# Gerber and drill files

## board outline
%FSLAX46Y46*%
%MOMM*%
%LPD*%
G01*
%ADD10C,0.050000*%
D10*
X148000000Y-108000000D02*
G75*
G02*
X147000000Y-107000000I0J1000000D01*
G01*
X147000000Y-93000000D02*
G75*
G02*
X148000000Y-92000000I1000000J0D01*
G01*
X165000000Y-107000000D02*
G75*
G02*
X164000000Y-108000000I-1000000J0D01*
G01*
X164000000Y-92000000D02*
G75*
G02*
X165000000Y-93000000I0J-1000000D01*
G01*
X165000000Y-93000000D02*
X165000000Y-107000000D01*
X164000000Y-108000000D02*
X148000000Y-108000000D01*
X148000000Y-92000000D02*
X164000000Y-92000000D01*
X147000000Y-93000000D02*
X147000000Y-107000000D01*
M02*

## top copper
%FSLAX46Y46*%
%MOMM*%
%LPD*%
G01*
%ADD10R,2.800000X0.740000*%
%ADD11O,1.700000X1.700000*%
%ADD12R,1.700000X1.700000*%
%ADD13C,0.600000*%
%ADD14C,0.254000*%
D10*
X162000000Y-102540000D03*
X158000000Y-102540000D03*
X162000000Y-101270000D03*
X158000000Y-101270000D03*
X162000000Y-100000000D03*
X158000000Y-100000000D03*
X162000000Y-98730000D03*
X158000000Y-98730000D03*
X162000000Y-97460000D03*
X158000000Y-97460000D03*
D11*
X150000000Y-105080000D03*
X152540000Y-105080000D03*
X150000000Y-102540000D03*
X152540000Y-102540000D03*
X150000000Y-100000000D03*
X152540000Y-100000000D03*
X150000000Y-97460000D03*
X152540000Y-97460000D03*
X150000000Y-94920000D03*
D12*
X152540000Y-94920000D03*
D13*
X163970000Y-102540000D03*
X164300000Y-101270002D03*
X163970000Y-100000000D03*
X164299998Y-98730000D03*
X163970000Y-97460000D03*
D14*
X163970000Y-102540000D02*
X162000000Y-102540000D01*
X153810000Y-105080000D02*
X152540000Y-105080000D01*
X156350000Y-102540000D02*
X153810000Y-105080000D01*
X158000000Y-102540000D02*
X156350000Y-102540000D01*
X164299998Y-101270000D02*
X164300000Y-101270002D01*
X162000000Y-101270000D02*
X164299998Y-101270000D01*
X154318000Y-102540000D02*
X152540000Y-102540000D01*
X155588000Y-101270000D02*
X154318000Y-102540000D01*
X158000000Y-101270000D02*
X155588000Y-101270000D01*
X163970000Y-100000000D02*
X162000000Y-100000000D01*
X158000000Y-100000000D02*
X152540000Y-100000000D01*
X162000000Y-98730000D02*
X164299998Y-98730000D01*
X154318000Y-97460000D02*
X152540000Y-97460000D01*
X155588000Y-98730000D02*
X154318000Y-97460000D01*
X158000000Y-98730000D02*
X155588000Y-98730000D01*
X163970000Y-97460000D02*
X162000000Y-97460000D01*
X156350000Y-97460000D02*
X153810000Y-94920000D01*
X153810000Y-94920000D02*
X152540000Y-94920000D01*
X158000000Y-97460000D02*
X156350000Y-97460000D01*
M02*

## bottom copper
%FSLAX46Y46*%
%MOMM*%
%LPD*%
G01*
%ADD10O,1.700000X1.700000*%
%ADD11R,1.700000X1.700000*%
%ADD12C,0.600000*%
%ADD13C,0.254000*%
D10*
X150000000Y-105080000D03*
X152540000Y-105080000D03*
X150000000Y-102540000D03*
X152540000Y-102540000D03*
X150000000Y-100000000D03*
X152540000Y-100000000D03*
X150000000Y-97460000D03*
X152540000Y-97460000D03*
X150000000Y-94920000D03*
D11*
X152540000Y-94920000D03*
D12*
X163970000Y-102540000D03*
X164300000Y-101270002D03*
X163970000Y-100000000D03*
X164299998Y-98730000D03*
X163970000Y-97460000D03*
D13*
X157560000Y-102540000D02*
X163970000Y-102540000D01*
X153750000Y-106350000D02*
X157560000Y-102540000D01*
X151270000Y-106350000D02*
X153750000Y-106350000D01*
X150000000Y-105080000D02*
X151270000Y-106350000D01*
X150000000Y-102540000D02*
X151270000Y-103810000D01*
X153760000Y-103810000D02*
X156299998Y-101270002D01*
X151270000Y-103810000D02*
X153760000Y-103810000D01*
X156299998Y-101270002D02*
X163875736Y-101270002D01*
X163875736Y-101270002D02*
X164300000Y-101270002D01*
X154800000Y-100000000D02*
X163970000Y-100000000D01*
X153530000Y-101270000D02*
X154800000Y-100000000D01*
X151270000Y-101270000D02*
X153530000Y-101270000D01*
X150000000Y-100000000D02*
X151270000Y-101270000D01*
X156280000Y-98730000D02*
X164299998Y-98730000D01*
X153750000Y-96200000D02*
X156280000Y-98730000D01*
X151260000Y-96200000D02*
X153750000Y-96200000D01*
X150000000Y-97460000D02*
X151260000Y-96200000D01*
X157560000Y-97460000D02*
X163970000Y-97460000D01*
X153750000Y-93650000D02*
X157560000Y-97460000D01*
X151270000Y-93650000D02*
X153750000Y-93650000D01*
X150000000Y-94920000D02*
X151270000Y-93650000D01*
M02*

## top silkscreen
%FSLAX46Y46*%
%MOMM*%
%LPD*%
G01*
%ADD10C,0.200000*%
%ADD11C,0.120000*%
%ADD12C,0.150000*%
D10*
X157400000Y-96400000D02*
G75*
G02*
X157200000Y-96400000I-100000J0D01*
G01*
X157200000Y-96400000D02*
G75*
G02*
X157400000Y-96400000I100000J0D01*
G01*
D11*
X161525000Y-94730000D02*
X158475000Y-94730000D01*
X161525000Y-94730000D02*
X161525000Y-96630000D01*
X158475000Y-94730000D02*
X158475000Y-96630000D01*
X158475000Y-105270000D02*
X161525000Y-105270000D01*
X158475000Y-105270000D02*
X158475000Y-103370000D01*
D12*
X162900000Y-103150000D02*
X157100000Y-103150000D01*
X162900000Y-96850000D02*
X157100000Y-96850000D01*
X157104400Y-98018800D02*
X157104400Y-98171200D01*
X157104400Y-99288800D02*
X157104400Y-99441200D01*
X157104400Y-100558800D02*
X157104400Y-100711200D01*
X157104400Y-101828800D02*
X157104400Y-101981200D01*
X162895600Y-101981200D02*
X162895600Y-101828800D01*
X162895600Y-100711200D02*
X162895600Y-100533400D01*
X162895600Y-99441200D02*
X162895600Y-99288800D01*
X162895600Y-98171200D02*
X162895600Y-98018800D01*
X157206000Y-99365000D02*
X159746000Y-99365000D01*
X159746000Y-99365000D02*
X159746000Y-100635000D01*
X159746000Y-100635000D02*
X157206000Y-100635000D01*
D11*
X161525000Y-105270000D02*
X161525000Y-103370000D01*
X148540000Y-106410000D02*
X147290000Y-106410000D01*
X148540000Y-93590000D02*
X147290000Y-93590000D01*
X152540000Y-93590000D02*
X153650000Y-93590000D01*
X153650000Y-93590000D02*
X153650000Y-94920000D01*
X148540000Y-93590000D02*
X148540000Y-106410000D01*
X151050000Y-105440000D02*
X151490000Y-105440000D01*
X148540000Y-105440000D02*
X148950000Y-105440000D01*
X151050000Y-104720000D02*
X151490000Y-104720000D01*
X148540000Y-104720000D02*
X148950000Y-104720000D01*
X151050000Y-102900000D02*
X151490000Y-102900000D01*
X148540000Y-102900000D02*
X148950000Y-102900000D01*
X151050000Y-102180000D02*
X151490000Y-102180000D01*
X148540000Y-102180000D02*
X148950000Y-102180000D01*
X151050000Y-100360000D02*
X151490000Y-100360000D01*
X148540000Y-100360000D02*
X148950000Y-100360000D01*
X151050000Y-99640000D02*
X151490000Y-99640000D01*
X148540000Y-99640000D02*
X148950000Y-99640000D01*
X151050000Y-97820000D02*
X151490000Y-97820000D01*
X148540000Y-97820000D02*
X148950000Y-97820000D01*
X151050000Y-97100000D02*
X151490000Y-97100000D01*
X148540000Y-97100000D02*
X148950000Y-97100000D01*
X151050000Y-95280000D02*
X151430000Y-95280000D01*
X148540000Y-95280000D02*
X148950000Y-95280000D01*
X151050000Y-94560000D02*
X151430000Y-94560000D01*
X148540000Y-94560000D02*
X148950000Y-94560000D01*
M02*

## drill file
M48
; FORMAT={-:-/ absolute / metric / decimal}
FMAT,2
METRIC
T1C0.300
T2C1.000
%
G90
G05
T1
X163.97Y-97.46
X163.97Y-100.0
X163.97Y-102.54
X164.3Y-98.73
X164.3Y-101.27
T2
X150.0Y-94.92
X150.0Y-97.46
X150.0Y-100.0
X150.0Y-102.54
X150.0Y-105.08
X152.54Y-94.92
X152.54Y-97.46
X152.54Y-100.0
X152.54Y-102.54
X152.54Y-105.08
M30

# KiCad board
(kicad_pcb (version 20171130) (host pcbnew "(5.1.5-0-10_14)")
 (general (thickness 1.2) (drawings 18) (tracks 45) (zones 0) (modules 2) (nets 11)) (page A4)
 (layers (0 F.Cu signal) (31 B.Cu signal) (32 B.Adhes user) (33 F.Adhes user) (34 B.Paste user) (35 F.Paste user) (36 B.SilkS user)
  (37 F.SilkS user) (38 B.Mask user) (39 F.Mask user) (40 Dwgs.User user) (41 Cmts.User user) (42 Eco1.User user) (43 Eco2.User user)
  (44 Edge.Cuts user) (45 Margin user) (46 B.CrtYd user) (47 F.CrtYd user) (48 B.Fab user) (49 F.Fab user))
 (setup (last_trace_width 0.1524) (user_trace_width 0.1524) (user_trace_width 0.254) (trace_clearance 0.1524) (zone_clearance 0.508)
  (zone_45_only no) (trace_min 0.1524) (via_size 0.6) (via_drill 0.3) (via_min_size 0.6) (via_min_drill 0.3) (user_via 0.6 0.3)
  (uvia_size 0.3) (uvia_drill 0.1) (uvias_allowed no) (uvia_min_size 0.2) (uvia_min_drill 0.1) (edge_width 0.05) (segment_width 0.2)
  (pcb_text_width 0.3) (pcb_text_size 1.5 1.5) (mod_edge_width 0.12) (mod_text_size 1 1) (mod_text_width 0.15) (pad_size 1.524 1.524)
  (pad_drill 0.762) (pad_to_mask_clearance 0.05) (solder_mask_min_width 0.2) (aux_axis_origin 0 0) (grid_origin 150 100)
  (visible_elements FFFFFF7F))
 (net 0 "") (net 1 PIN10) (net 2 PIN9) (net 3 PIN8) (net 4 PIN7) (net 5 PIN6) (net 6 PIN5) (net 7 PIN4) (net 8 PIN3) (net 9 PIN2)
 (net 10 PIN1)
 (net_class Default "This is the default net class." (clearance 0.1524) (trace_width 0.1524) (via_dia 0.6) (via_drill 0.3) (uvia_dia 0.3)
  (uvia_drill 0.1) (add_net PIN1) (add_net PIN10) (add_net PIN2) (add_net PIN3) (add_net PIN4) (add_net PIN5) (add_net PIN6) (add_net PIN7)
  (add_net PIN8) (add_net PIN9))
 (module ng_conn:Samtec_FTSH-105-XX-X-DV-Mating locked (layer F.Cu) (at 160 100 90)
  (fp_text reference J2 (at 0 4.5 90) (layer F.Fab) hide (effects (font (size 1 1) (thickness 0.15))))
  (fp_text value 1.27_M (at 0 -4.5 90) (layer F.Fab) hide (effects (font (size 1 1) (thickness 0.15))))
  (fp_circle (center 3.6 -2.7) (end 3.7 -2.7) (layer F.SilkS) (width 0.2))
  (fp_line (start 5.27 1.525) (end 5.27 -1.525) (layer F.SilkS) (width 0.12))
  (fp_line (start 5.27 1.525) (end 3.37 1.525) (layer F.SilkS) (width 0.12))
  (fp_line (start 5.27 -1.525) (end 3.37 -1.525) (layer F.SilkS) (width 0.12))
  (fp_line (start -5.27 -1.525) (end -5.27 1.525) (layer F.SilkS) (width 0.12))
  (fp_line (start -5.27 -1.525) (end -3.37 -1.525) (layer F.SilkS) (width 0.12))
  (fp_line (start -3.15 2.9) (end -3.15 -2.9) (layer F.SilkS) (width 0.15))
  (fp_line (start 3.15 2.9) (end 3.15 -2.9) (layer F.SilkS) (width 0.15))
  (fp_line (start 1.9812 -2.8956) (end 1.8288 -2.8956) (layer F.SilkS) (width 0.15))
  (fp_line (start 0.7112 -2.8956) (end 0.5588 -2.8956) (layer F.SilkS) (width 0.15))
  (fp_line (start -0.5588 -2.8956) (end -0.7112 -2.8956) (layer F.SilkS) (width 0.15))
  (fp_line (start -1.8288 -2.8956) (end -1.9812 -2.8956) (layer F.SilkS) (width 0.15))
  (fp_line (start -1.9812 2.8956) (end -1.8288 2.8956) (layer F.SilkS) (width 0.15))
  (fp_line (start -0.7112 2.8956) (end -0.5334 2.8956) (layer F.SilkS) (width 0.15))
  (fp_line (start 0.5588 2.8956) (end 0.7112 2.8956) (layer F.SilkS) (width 0.15))
  (fp_line (start 1.8288 2.8956) (end 1.9812 2.8956) (layer F.SilkS) (width 0.15))
  (fp_line (start 0.635 -2.794) (end 0.635 -0.254) (layer F.SilkS) (width 0.15))
  (fp_line (start 0.635 -0.254) (end -0.635 -0.254) (layer F.SilkS) (width 0.15))
  (fp_line (start -0.635 -0.254) (end -0.635 -2.794) (layer F.SilkS) (width 0.15))
  (fp_line (start -5.27 1.525) (end -3.37 1.525) (layer F.SilkS) (width 0.12))
  (pad 10 smd rect (at -2.54 2 270) (size 0.74 2.8) (layers F.Cu F.Paste F.Mask) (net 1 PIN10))
  (pad 9 smd rect (at -2.54 -2 270) (size 0.74 2.8) (layers F.Cu F.Paste F.Mask) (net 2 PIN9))
  (pad 8 smd rect (at -1.27 2 270) (size 0.74 2.8) (layers F.Cu F.Paste F.Mask) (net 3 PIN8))
  (pad 7 smd rect (at -1.27 -2 270) (size 0.74 2.8) (layers F.Cu F.Paste F.Mask) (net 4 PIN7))
  (pad 6 smd rect (at 0 2 270) (size 0.74 2.8) (layers F.Cu F.Paste F.Mask) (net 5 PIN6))
  (pad 5 smd rect (at 0 -2 270) (size 0.74 2.8) (layers F.Cu F.Paste F.Mask) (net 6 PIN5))
  (pad 4 smd rect (at 1.27 2 270) (size 0.74 2.8) (layers F.Cu F.Paste F.Mask) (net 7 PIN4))
  (pad 3 smd rect (at 1.27 -2 270) (size 0.74 2.8) (layers F.Cu F.Paste F.Mask) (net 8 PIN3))
  (pad 2 smd rect (at 2.54 2 270) (size 0.74 2.8) (layers F.Cu F.Paste F.Mask) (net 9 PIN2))
  (pad 1 smd rect (at 2.54 -2 270) (size 0.74 2.8) (layers F.Cu F.Paste F.Mask) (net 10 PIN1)))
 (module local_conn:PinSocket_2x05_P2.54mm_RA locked (layer F.Cu) (at 152.54 94.92)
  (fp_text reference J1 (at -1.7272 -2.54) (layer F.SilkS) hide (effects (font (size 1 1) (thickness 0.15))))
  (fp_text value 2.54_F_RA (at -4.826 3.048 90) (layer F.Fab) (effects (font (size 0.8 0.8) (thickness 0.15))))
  (fp_line (start -4 11.49) (end -5.25 11.49) (layer F.SilkS) (width 0.12))
  (fp_line (start -4 -1.33) (end -5.25 -1.33) (layer F.SilkS) (width 0.12))
  (fp_line (start 0 -1.33) (end 1.11 -1.33) (layer F.SilkS) (width 0.12))
  (fp_line (start 1.11 -1.33) (end 1.11 0) (layer F.SilkS) (width 0.12))
  (fp_line (start -4 -1.33) (end -4 11.49) (layer F.SilkS) (width 0.12))
  (fp_line (start -1.49 10.52) (end -1.05 10.52) (layer F.SilkS) (width 0.12))
  (fp_line (start -4 10.52) (end -3.59 10.52) (layer F.SilkS) (width 0.12))
  (fp_line (start -1.49 9.8) (end -1.05 9.8) (layer F.SilkS) (width 0.12))
  (fp_line (start -4 9.8) (end -3.59 9.8) (layer F.SilkS) (width 0.12))
  (fp_line (start -1.49 7.98) (end -1.05 7.98) (layer F.SilkS) (width 0.12))
  (fp_line (start -4 7.98) (end -3.59 7.98) (layer F.SilkS) (width 0.12))
  (fp_line (start -1.49 7.26) (end -1.05 7.26) (layer F.SilkS) (width 0.12))
  (fp_line (start -4 7.26) (end -3.59 7.26) (layer F.SilkS) (width 0.12))
  (fp_line (start -1.49 5.44) (end -1.05 5.44) (layer F.SilkS) (width 0.12))
  (fp_line (start -4 5.44) (end -3.59 5.44) (layer F.SilkS) (width 0.12))
  (fp_line (start -1.49 4.72) (end -1.05 4.72) (layer F.SilkS) (width 0.12))
  (fp_line (start -4 4.72) (end -3.59 4.72) (layer F.SilkS) (width 0.12))
  (fp_line (start -1.49 2.9) (end -1.05 2.9) (layer F.SilkS) (width 0.12))
  (fp_line (start -4 2.9) (end -3.59 2.9) (layer F.SilkS) (width 0.12))
  (fp_line (start -1.49 2.18) (end -1.05 2.18) (layer F.SilkS) (width 0.12))
  (fp_line (start -4 2.18) (end -3.59 2.18) (layer F.SilkS) (width 0.12))
  (fp_line (start -1.49 0.36) (end -1.11 0.36) (layer F.SilkS) (width 0.12))
  (fp_line (start -4 0.36) (end -3.59 0.36) (layer F.SilkS) (width 0.12))
  (fp_line (start -1.49 -0.36) (end -1.11 -0.36) (layer F.SilkS) (width 0.12))
  (fp_line (start -4 -0.36) (end -3.59 -0.36) (layer F.SilkS) (width 0.12))
  (pad 10 thru_hole oval (at -2.54 10.16) (size 1.7 1.7) (drill 1) (layers *.Cu *.Mask) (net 1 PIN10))
  (pad 9 thru_hole oval (at 0 10.16) (size 1.7 1.7) (drill 1) (layers *.Cu *.Mask) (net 2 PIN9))
  (pad 8 thru_hole oval (at -2.54 7.62) (size 1.7 1.7) (drill 1) (layers *.Cu *.Mask) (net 3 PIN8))
  (pad 7 thru_hole oval (at 0 7.62) (size 1.7 1.7) (drill 1) (layers *.Cu *.Mask) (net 4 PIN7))
  (pad 6 thru_hole oval (at -2.54 5.08) (size 1.7 1.7) (drill 1) (layers *.Cu *.Mask) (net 5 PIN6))
  (pad 5 thru_hole oval (at 0 5.08) (size 1.7 1.7) (drill 1) (layers *.Cu *.Mask) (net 6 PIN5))
  (pad 4 thru_hole oval (at -2.54 2.54) (size 1.7 1.7) (drill 1) (layers *.Cu *.Mask) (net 7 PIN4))
  (pad 3 thru_hole oval (at 0 2.54) (size 1.7 1.7) (drill 1) (layers *.Cu *.Mask) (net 8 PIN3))
  (pad 2 thru_hole oval (at -2.54 0) (size 1.7 1.7) (drill 1) (layers *.Cu *.Mask) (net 9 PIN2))
  (pad 1 thru_hole rect (at 0 0) (size 1.7 1.7) (drill 1) (layers *.Cu *.Mask) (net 10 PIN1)))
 (gr_arc (start 148 107) (end 147 107) (angle -90) (layer Edge.Cuts) (width 0.05))
 (gr_arc (start 148 93) (end 148 92) (angle -90) (layer Edge.Cuts) (width 0.05))
 (gr_arc (start 164 107) (end 164 108) (angle -90) (layer Edge.Cuts) (width 0.05))
 (gr_arc (start 164 93) (end 165 93) (angle -90) (layer Edge.Cuts) (width 0.05))
 (gr_line (start 165 93) (end 165 107) (layer Edge.Cuts) (width 0.05))
 (gr_line (start 164 108) (end 148 108) (layer Edge.Cuts) (width 0.05))
 (gr_line (start 148 92) (end 164 92) (layer Edge.Cuts) (width 0.05))
 (gr_line (start 147 93) (end 147 107) (layer Edge.Cuts) (width 0.05))
 (via (at 163.97 102.54) (size 0.6) (drill 0.3) (layers F.Cu B.Cu) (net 1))
 (segment (start 163.97 102.54) (end 162 102.54) (width 0.254) (layer F.Cu) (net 1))
 (segment (start 157.56 102.54) (end 163.97 102.54) (width 0.254) (layer B.Cu) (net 1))
 (segment (start 153.75 106.35) (end 157.56 102.54) (width 0.254) (layer B.Cu) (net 1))
 (segment (start 151.27 106.35) (end 153.75 106.35) (width 0.254) (layer B.Cu) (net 1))
 (segment (start 150 105.08) (end 151.27 106.35) (width 0.254) (layer B.Cu) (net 1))
 (segment (start 153.81 105.08) (end 152.54 105.08) (width 0.254) (layer F.Cu) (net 2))
 (segment (start 156.35 102.54) (end 153.81 105.08) (width 0.254) (layer F.Cu) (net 2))
 (segment (start 158 102.54) (end 156.35 102.54) (width 0.254) (layer F.Cu) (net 2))
 (via (at 164.3 101.270002) (size 0.6) (drill 0.3) (layers F.Cu B.Cu) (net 3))
 (segment (start 164.299998 101.27) (end 164.3 101.270002) (width 0.254) (layer F.Cu) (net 3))
 (segment (start 162 101.27) (end 164.299998 101.27) (width 0.254) (layer F.Cu) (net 3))
 (segment (start 150 102.54) (end 151.27 103.81) (width 0.254) (layer B.Cu) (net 3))
 (segment (start 153.76 103.81) (end 156.299998 101.270002) (width 0.254) (layer B.Cu) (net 3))
 (segment (start 151.27 103.81) (end 153.76 103.81) (width 0.254) (layer B.Cu) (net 3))
 (segment (start 156.299998 101.270002) (end 163.875736 101.270002) (width 0.254) (layer B.Cu) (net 3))
 (segment (start 163.875736 101.270002) (end 164.3 101.270002) (width 0.254) (layer B.Cu) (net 3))
 (segment (start 154.318 102.54) (end 152.54 102.54) (width 0.254) (layer F.Cu) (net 4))
 (segment (start 155.588 101.27) (end 154.318 102.54) (width 0.254) (layer F.Cu) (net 4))
 (segment (start 158 101.27) (end 155.588 101.27) (width 0.254) (layer F.Cu) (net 4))
 (via (at 163.97 100) (size 0.6) (drill 0.3) (layers F.Cu B.Cu) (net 5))
 (segment (start 163.97 100) (end 162 100) (width 0.254) (layer F.Cu) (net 5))
 (segment (start 154.8 100) (end 163.97 100) (width 0.254) (layer B.Cu) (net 5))
 (segment (start 153.53 101.27) (end 154.8 100) (width 0.254) (layer B.Cu) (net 5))
 (segment (start 151.27 101.27) (end 153.53 101.27) (width 0.254) (layer B.Cu) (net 5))
 (segment (start 150 100) (end 151.27 101.27) (width 0.254) (layer B.Cu) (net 5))
 (segment (start 158 100) (end 152.54 100) (width 0.254) (layer F.Cu) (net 6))
 (via (at 164.299998 98.73) (size 0.6) (drill 0.3) (layers F.Cu B.Cu) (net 7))
 (segment (start 162 98.73) (end 164.299998 98.73) (width 0.254) (layer F.Cu) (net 7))
 (segment (start 156.28 98.73) (end 164.299998 98.73) (width 0.254) (layer B.Cu) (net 7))
 (segment (start 153.75 96.2) (end 156.28 98.73) (width 0.254) (layer B.Cu) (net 7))
 (segment (start 151.26 96.2) (end 153.75 96.2) (width 0.254) (layer B.Cu) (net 7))
 (segment (start 150 97.46) (end 151.26 96.2) (width 0.254) (layer B.Cu) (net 7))
 (segment (start 154.318 97.46) (end 152.54 97.46) (width 0.254) (layer F.Cu) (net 8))
 (segment (start 155.588 98.73) (end 154.318 97.46) (width 0.254) (layer F.Cu) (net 8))
 (segment (start 158 98.73) (end 155.588 98.73) (width 0.254) (layer F.Cu) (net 8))
 (via (at 163.97 97.46) (size 0.6) (drill 0.3) (layers F.Cu B.Cu) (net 9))
 (segment (start 163.97 97.46) (end 162 97.46) (width 0.254) (layer F.Cu) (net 9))
 (segment (start 157.56 97.46) (end 163.97 97.46) (width 0.254) (layer B.Cu) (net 9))
 (segment (start 153.75 93.65) (end 157.56 97.46) (width 0.254) (layer B.Cu) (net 9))
 (segment (start 151.27 93.65) (end 153.75 93.65) (width 0.254) (layer B.Cu) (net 9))
 (segment (start 150 94.92) (end 151.27 93.65) (width 0.254) (layer B.Cu) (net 9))
 (segment (start 156.35 97.46) (end 153.81 94.92) (width 0.254) (layer F.Cu) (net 10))
 (segment (start 153.81 94.92) (end 152.54 94.92) (width 0.254) (layer F.Cu) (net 10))
 (segment (start 158 97.46) (end 156.35 97.46) (width 0.254) (layer F.Cu) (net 10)))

